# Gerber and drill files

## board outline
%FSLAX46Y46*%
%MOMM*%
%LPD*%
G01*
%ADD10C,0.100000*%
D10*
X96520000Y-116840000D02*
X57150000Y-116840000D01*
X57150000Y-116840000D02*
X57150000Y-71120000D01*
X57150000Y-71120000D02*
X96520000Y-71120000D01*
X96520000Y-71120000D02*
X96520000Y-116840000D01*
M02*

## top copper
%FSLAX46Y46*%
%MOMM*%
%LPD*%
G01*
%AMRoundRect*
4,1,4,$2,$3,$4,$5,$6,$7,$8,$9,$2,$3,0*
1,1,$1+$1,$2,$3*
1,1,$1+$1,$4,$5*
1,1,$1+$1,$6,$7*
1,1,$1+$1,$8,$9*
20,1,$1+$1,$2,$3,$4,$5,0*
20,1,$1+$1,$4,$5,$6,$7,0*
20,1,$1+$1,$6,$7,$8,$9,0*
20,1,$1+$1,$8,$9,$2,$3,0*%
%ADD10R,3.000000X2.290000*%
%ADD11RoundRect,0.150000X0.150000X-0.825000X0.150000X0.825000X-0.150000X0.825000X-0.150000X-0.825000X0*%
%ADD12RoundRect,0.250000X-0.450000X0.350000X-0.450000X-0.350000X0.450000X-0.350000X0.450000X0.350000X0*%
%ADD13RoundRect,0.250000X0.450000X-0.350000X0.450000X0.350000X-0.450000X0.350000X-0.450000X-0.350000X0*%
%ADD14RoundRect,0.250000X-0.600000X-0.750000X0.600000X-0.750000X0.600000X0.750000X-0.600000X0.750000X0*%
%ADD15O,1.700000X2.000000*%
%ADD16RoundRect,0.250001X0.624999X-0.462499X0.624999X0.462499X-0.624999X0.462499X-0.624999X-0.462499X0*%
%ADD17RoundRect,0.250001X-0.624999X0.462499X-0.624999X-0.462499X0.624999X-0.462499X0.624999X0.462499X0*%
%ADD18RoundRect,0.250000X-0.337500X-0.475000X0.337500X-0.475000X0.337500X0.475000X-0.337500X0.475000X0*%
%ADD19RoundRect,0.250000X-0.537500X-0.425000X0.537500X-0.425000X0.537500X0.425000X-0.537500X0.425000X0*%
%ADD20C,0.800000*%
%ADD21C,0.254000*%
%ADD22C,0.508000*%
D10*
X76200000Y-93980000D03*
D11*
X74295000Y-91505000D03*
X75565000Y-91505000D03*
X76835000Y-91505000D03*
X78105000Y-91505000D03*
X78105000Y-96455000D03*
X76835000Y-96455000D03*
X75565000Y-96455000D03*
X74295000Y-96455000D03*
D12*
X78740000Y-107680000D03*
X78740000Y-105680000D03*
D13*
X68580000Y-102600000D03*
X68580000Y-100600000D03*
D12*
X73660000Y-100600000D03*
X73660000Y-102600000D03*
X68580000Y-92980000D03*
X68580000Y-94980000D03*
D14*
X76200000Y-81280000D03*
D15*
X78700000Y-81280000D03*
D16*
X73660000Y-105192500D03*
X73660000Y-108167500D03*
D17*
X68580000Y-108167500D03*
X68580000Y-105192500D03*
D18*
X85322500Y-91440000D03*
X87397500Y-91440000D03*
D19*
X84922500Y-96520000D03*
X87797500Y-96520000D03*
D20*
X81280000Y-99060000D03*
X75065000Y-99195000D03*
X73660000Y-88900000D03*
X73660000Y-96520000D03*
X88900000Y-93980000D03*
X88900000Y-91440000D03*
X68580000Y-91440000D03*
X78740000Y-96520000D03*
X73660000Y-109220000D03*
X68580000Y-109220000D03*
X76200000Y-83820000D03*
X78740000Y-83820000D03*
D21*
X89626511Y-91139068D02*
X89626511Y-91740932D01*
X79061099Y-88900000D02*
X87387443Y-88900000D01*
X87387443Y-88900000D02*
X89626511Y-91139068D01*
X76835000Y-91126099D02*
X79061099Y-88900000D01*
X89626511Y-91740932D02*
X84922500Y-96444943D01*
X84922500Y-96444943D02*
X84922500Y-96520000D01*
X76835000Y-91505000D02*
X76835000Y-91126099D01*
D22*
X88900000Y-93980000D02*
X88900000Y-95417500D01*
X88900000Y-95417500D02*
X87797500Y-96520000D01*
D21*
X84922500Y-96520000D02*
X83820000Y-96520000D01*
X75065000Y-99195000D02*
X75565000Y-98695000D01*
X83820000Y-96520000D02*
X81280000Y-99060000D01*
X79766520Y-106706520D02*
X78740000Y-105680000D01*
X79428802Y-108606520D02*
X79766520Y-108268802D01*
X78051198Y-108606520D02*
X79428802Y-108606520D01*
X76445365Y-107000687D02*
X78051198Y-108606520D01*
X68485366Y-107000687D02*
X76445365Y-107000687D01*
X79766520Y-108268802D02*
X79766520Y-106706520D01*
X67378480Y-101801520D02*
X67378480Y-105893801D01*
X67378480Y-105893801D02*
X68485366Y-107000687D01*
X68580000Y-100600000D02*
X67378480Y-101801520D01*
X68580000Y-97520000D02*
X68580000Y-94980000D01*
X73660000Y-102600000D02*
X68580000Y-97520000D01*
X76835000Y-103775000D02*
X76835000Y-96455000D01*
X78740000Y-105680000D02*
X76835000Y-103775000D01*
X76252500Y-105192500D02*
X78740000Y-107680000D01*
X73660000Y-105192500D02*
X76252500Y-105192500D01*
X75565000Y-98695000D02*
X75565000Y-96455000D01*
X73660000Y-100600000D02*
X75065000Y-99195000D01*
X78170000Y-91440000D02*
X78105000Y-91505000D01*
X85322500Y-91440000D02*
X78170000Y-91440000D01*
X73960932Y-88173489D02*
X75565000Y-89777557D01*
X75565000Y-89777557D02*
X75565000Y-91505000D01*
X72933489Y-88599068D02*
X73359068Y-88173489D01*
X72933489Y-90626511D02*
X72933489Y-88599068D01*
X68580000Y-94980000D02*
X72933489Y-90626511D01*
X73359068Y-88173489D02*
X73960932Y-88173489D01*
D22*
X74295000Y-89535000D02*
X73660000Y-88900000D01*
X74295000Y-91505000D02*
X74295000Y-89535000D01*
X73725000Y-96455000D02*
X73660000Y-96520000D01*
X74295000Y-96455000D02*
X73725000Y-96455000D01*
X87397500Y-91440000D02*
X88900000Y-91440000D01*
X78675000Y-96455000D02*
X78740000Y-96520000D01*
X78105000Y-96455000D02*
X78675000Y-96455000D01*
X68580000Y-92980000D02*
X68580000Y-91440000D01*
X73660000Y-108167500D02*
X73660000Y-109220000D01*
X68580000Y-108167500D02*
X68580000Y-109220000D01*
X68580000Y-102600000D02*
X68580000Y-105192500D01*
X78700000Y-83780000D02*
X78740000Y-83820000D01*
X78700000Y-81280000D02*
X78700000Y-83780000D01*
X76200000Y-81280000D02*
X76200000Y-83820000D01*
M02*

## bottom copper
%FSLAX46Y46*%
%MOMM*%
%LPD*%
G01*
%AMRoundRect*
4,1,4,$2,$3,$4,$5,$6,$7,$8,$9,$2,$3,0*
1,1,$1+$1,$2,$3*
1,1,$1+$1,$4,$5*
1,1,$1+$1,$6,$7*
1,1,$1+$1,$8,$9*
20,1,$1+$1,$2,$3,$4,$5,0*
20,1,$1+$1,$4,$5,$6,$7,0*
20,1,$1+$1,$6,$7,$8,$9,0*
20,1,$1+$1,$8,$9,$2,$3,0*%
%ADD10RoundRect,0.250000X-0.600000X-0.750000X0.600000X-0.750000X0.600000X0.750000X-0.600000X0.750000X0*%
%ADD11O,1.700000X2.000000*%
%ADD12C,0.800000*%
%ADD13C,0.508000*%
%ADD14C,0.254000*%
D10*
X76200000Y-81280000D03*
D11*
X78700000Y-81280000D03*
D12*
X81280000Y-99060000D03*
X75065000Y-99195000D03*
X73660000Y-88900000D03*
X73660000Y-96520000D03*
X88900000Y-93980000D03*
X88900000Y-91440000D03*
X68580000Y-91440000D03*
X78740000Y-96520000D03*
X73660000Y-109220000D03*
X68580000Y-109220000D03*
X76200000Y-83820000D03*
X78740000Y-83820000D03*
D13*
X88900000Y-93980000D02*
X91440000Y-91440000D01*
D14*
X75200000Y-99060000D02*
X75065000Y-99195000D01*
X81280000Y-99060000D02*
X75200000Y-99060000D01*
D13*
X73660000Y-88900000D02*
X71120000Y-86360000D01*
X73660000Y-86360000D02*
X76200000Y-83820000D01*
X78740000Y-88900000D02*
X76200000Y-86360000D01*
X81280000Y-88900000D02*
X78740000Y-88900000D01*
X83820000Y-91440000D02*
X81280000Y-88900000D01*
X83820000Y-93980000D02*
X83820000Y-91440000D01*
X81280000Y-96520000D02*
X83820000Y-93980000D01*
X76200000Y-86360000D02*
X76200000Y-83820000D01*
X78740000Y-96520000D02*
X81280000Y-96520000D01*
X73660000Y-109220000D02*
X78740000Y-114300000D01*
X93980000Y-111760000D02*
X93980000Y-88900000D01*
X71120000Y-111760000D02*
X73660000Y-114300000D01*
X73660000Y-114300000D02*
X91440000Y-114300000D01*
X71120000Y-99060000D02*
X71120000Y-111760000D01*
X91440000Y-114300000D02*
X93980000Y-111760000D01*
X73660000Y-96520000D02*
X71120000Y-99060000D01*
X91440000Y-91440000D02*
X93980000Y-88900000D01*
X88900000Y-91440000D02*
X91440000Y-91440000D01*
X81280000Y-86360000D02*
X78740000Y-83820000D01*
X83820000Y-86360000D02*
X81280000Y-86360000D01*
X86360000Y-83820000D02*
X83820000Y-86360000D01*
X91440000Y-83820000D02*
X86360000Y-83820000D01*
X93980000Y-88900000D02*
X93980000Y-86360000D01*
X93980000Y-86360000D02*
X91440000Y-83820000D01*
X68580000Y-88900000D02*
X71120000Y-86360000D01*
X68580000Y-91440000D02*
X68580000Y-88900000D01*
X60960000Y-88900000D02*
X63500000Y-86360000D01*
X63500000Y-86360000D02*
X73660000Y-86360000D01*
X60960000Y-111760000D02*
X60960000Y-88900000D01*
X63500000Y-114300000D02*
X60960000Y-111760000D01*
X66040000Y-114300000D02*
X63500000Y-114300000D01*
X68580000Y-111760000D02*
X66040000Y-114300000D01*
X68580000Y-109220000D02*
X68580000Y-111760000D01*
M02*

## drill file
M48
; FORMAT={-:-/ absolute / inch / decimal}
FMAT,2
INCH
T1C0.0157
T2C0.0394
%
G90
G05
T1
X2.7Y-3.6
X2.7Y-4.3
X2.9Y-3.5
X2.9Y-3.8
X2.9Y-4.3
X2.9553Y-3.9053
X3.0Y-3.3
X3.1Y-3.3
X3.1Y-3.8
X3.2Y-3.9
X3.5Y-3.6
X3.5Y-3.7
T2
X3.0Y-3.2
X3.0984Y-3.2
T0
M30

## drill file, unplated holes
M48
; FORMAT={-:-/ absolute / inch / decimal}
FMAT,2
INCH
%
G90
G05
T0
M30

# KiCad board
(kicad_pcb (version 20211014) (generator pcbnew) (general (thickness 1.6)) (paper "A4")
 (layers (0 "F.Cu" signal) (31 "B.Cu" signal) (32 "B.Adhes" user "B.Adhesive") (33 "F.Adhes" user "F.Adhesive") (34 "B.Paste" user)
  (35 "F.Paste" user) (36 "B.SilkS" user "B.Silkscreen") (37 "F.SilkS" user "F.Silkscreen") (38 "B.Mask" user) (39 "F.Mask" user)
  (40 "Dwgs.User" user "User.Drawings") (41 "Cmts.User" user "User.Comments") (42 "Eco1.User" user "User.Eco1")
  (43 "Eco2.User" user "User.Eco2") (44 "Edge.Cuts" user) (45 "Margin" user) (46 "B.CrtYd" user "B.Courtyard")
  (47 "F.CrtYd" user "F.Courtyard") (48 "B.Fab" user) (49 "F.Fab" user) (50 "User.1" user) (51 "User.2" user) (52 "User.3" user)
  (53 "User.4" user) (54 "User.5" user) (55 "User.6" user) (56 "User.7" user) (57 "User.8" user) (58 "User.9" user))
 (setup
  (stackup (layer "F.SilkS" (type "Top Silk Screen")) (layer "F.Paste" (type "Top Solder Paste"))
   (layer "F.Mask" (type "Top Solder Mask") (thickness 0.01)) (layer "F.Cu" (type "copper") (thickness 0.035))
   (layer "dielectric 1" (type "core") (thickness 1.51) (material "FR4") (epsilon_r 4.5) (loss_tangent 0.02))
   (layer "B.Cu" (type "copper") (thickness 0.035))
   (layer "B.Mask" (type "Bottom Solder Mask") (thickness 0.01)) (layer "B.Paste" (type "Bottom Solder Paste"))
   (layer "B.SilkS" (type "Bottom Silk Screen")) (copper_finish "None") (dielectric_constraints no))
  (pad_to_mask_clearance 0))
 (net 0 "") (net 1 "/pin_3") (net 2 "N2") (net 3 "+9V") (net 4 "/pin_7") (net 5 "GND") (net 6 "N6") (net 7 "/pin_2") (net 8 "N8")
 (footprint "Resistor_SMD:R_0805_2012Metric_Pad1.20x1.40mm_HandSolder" (layer "F.Cu") (at 78.74 106.68 -90)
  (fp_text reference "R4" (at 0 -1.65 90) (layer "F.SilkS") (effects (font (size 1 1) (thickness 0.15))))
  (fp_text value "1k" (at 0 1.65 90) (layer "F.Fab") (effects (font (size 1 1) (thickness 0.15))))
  (pad "1" smd roundrect (at -1 0 270) (size 1.2 1.4) (layers "F.Cu" "F.Paste" "F.Mask") (roundrect_rratio 0.2083333333) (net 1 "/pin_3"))
  (pad "2" smd roundrect (at 1 0 270) (size 1.2 1.4) (layers "F.Cu" "F.Paste" "F.Mask") (roundrect_rratio 0.2083333333) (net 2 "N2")))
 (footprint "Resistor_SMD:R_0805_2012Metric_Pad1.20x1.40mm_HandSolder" (layer "F.Cu") (at 68.58 93.98 -90)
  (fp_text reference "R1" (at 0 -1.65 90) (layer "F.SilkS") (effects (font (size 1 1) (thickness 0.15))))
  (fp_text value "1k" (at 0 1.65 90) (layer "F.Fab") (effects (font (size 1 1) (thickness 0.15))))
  (pad "1" smd roundrect (at -1 0 270) (size 1.2 1.4) (layers "F.Cu" "F.Paste" "F.Mask") (roundrect_rratio 0.2083333333) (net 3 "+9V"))
  (pad "2" smd roundrect (at 1 0 270) (size 1.2 1.4) (layers "F.Cu" "F.Paste" "F.Mask") (roundrect_rratio 0.2083333333) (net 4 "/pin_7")))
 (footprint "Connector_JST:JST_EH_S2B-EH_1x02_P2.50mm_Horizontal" (layer "F.Cu") (at 76.2 81.28)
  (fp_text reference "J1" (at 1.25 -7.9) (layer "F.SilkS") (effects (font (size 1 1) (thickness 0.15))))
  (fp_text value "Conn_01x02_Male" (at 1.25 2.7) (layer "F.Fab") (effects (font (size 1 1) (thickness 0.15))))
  (pad "1" thru_hole roundrect (at 0 0) (size 1.7 2) (drill 1) (layers *.Cu *.Mask) (roundrect_rratio 0.1470588235) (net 3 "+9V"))
  (pad "2" thru_hole oval (at 2.5 0) (size 1.7 2) (drill 1) (layers *.Cu *.Mask) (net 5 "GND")))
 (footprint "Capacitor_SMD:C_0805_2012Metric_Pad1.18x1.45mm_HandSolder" (layer "F.Cu") (at 86.36 91.44)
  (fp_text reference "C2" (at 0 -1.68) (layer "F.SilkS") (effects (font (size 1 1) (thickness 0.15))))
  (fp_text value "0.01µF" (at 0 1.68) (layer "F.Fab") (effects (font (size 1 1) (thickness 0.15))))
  (pad "1" smd roundrect (at -1.0375 0) (size 1.175 1.45) (layers "F.Cu" "F.Paste" "F.Mask") (roundrect_rratio 0.2127659574) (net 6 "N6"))
  (pad "2" smd roundrect (at 1.0375 0) (size 1.175 1.45) (layers "F.Cu" "F.Paste" "F.Mask") (roundrect_rratio 0.2127659574) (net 5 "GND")))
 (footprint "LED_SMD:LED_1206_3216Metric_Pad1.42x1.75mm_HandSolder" (layer "F.Cu") (at 73.66 106.68 90)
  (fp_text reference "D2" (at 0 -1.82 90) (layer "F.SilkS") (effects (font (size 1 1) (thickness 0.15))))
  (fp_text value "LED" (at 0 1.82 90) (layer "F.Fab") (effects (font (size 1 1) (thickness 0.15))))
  (pad "1" smd roundrect (at -1.4875 0 90) (size 1.425 1.75) (layers "F.Cu" "F.Paste" "F.Mask") (roundrect_rratio 0.1754392982)
   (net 5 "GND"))
  (pad "2" smd roundrect (at 1.4875 0 90) (size 1.425 1.75) (layers "F.Cu" "F.Paste" "F.Mask") (roundrect_rratio 0.1754392982) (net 2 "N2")))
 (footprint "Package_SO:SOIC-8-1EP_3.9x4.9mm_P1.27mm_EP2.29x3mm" (layer "F.Cu") (at 76.2 93.98 90)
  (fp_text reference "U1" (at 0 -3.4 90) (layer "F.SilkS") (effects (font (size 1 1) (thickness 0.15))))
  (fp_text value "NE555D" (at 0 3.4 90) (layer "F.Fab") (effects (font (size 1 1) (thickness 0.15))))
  (pad "" smd roundrect (at 0.57 -0.75 90) (size 0.92 1.21) (layers "F.Paste") (roundrect_rratio 0.25))
  (pad "" smd roundrect (at 0.57 0.75 90) (size 0.92 1.21) (layers "F.Paste") (roundrect_rratio 0.25))
  (pad "" smd roundrect (at -0.57 -0.75 90) (size 0.92 1.21) (layers "F.Paste") (roundrect_rratio 0.25))
  (pad "" smd roundrect (at -0.57 0.75 90) (size 0.92 1.21) (layers "F.Paste") (roundrect_rratio 0.25))
  (pad "1" smd roundrect (at -2.475 -1.905 90) (size 1.95 0.6) (layers "F.Cu" "F.Paste" "F.Mask") (roundrect_rratio 0.25) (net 5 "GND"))
  (pad "2" smd roundrect (at -2.475 -0.635 90) (size 1.95 0.6) (layers "F.Cu" "F.Paste" "F.Mask") (roundrect_rratio 0.25) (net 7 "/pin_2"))
  (pad "3" smd roundrect (at -2.475 0.635 90) (size 1.95 0.6) (layers "F.Cu" "F.Paste" "F.Mask") (roundrect_rratio 0.25) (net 1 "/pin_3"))
  (pad "4" smd roundrect (at -2.475 1.905 90) (size 1.95 0.6) (layers "F.Cu" "F.Paste" "F.Mask") (roundrect_rratio 0.25) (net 3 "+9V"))
  (pad "5" smd roundrect (at 2.475 1.905 90) (size 1.95 0.6) (layers "F.Cu" "F.Paste" "F.Mask") (roundrect_rratio 0.25) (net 6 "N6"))
  (pad "6" smd roundrect (at 2.475 0.635 90) (size 1.95 0.6) (layers "F.Cu" "F.Paste" "F.Mask") (roundrect_rratio 0.25) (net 7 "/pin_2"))
  (pad "7" smd roundrect (at 2.475 -0.635 90) (size 1.95 0.6) (layers "F.Cu" "F.Paste" "F.Mask") (roundrect_rratio 0.25) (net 4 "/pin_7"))
  (pad "8" smd roundrect (at 2.475 -1.905 90) (size 1.95 0.6) (layers "F.Cu" "F.Paste" "F.Mask") (roundrect_rratio 0.25) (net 3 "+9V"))
  (pad "9" smd rect (at 0 0 90) (size 2.29 3) (layers "F.Cu" "F.Mask")))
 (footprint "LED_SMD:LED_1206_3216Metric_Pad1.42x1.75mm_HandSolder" (layer "F.Cu") (at 68.58 106.68 -90)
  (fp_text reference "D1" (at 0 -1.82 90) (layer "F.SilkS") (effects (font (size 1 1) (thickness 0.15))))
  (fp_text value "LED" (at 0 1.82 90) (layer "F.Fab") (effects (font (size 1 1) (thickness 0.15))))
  (pad "1" smd roundrect (at -1.4875 0 270) (size 1.425 1.75) (layers "F.Cu" "F.Paste" "F.Mask") (roundrect_rratio 0.1754392982)
   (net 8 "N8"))
  (pad "2" smd roundrect (at 1.4875 0 270) (size 1.425 1.75) (layers "F.Cu" "F.Paste" "F.Mask") (roundrect_rratio 0.1754392982)
   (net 3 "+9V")))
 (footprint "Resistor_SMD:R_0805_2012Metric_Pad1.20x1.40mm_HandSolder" (layer "F.Cu") (at 68.58 101.6 90)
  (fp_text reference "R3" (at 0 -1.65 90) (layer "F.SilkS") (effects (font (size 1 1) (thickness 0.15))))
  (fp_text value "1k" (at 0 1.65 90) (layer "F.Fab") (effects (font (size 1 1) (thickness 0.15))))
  (pad "1" smd roundrect (at -1 0 90) (size 1.2 1.4) (layers "F.Cu" "F.Paste" "F.Mask") (roundrect_rratio 0.2083333333) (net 8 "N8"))
  (pad "2" smd roundrect (at 1 0 90) (size 1.2 1.4) (layers "F.Cu" "F.Paste" "F.Mask") (roundrect_rratio 0.2083333333) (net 1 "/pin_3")))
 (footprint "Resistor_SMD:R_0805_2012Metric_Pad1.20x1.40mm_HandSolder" (layer "F.Cu") (at 73.66 101.6 -90)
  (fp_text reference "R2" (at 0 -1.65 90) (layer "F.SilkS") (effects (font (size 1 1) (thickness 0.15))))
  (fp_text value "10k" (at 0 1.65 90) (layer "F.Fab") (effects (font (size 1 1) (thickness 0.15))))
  (pad "1" smd roundrect (at -1 0 270) (size 1.2 1.4) (layers "F.Cu" "F.Paste" "F.Mask") (roundrect_rratio 0.2083333333) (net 7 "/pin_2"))
  (pad "2" smd roundrect (at 1 0 270) (size 1.2 1.4) (layers "F.Cu" "F.Paste" "F.Mask") (roundrect_rratio 0.2083333333) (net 4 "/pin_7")))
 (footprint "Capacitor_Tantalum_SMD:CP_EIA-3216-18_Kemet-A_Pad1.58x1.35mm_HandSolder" (layer "F.Cu") (at 86.36 96.52)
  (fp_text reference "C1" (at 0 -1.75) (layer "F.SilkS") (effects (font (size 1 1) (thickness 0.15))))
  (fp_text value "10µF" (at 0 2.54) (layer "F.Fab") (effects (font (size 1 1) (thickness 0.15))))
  (pad "1" smd roundrect (at -1.4375 0) (size 1.575 1.35) (layers "F.Cu" "F.Paste" "F.Mask") (roundrect_rratio 0.1851851852)
   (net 7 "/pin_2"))
  (pad "2" smd roundrect (at 1.4375 0) (size 1.575 1.35) (layers "F.Cu" "F.Paste" "F.Mask") (roundrect_rratio 0.1851851852) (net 5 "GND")))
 (gr_rect (start 96.52 116.84) (end 57.15 71.12) (layer "Edge.Cuts") (width 0.1) (fill none))
 (segment (start 84.9225 96.52) (end 83.82 96.52) (width 0.254) (layer "F.Cu") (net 7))
 (segment (start 89.626511 91.139068) (end 89.626511 91.740932) (width 0.254) (layer "F.Cu") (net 7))
 (segment (start 84.9225 96.444943) (end 84.9225 96.52) (width 0.254) (layer "F.Cu") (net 7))
 (segment (start 73.66 100.6) (end 75.065 99.195) (width 0.254) (layer "F.Cu") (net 7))
 (segment (start 76.835 91.126099) (end 79.061099 88.9) (width 0.254) (layer "F.Cu") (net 7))
 (segment (start 87.387443 88.9) (end 89.626511 91.139068) (width 0.254) (layer "F.Cu") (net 7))
 (segment (start 75.565 98.695) (end 75.565 96.455) (width 0.254) (layer "F.Cu") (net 7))
 (segment (start 89.626511 91.740932) (end 84.9225 96.444943) (width 0.254) (layer "F.Cu") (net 7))
 (segment (start 79.061099 88.9) (end 87.387443 88.9) (width 0.254) (layer "F.Cu") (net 7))
 (segment (start 75.065 99.195) (end 75.565 98.695) (width 0.254) (layer "F.Cu") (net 7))
 (segment (start 83.82 96.52) (end 81.28 99.06) (width 0.254) (layer "F.Cu") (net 7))
 (segment (start 76.835 91.505) (end 76.835 91.126099) (width 0.254) (layer "F.Cu") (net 7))
 (via (at 75.065 99.195) (size 0.8) (drill 0.4) (layers "F.Cu" "B.Cu") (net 7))
 (via (at 81.28 99.06) (size 0.8) (drill 0.4) (layers "F.Cu" "B.Cu") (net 7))
 (segment (start 75.2 99.06) (end 75.065 99.195) (width 0.254) (layer "B.Cu") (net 7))
 (segment (start 81.28 99.06) (end 75.2 99.06) (width 0.254) (layer "B.Cu") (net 7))
 (segment (start 73.725 96.455) (end 73.66 96.52) (width 0.508) (layer "F.Cu") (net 5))
 (segment (start 78.7 83.78) (end 78.74 83.82) (width 0.508) (layer "F.Cu") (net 5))
 (segment (start 87.3975 91.44) (end 88.9 91.44) (width 0.508) (layer "F.Cu") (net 5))
 (segment (start 78.7 81.28) (end 78.7 83.78) (width 0.508) (layer "F.Cu") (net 5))
 (segment (start 88.9 95.4175) (end 87.7975 96.52) (width 0.508) (layer "F.Cu") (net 5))
 (segment (start 73.66 108.1675) (end 73.66 109.22) (width 0.508) (layer "F.Cu") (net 5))
 (segment (start 88.9 93.98) (end 88.9 95.4175) (width 0.508) (layer "F.Cu") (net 5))
 (segment (start 74.295 96.455) (end 73.725 96.455) (width 0.508) (layer "F.Cu") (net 5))
 (via (at 78.74 83.82) (size 0.8) (drill 0.4) (layers "F.Cu" "B.Cu") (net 5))
 (via (at 88.9 91.44) (size 0.8) (drill 0.4) (layers "F.Cu" "B.Cu") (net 5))
 (via (at 73.66 109.22) (size 0.8) (drill 0.4) (layers "F.Cu" "B.Cu") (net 5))
 (via (at 73.66 96.52) (size 0.8) (drill 0.4) (layers "F.Cu" "B.Cu") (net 5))
 (via (at 88.9 93.98) (size 0.8) (drill 0.4) (layers "F.Cu" "B.Cu") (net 5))
 (segment (start 88.9 91.44) (end 91.44 91.44) (width 0.508) (layer "B.Cu") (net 5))
 (segment (start 93.98 111.76) (end 93.98 88.9) (width 0.508) (layer "B.Cu") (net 5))
 (segment (start 73.66 109.22) (end 78.74 114.3) (width 0.508) (layer "B.Cu") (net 5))
 (segment (start 71.12 111.76) (end 73.66 114.3) (width 0.508) (layer "B.Cu") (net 5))
 (segment (start 88.9 93.98) (end 91.44 91.44) (width 0.508) (layer "B.Cu") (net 5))
 (segment (start 73.66 96.52) (end 71.12 99.06) (width 0.508) (layer "B.Cu") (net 5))
 (segment (start 93.98 88.9) (end 93.98 86.36) (width 0.508) (layer "B.Cu") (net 5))
 (segment (start 71.12 99.06) (end 71.12 111.76) (width 0.508) (layer "B.Cu") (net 5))
 (segment (start 86.36 83.82) (end 83.82 86.36) (width 0.508) (layer "B.Cu") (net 5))
 (segment (start 91.44 91.44) (end 93.98 88.9) (width 0.508) (layer "B.Cu") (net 5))
 (segment (start 93.98 86.36) (end 91.44 83.82) (width 0.508) (layer "B.Cu") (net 5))
 (segment (start 81.28 86.36) (end 78.74 83.82) (width 0.508) (layer "B.Cu") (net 5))
 (segment (start 73.66 114.3) (end 91.44 114.3) (width 0.508) (layer "B.Cu") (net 5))
 (segment (start 83.82 86.36) (end 81.28 86.36) (width 0.508) (layer "B.Cu") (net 5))
 (segment (start 91.44 114.3) (end 93.98 111.76) (width 0.508) (layer "B.Cu") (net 5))
 (segment (start 91.44 83.82) (end 86.36 83.82) (width 0.508) (layer "B.Cu") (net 5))
 (segment (start 78.17 91.44) (end 78.105 91.505) (width 0.254) (layer "F.Cu") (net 6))
 (segment (start 85.3225 91.44) (end 78.17 91.44) (width 0.254) (layer "F.Cu") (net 6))
 (segment (start 68.58 102.6) (end 68.58 105.1925) (width 0.508) (layer "F.Cu") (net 8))
 (segment (start 78.105 96.455) (end 78.675 96.455) (width 0.508) (layer "F.Cu") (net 3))
 (segment (start 76.2 81.28) (end 76.2 83.82) (width 0.508) (layer "F.Cu") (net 3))
 (segment (start 78.675 96.455) (end 78.74 96.52) (width 0.508) (layer "F.Cu") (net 3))
 (segment (start 74.295 89.535) (end 73.66 88.9) (width 0.508) (layer "F.Cu") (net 3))
 (segment (start 68.58 92.98) (end 68.58 91.44) (width 0.508) (layer "F.Cu") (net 3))
 (segment (start 68.58 108.1675) (end 68.58 109.22) (width 0.508) (layer "F.Cu") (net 3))
 (segment (start 74.295 91.505) (end 74.295 89.535) (width 0.508) (layer "F.Cu") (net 3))
 (via (at 68.58 91.44) (size 0.8) (drill 0.4) (layers "F.Cu" "B.Cu") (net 3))
 (via (at 73.66 88.9) (size 0.8) (drill 0.4) (layers "F.Cu" "B.Cu") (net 3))
 (via (at 76.2 83.82) (size 0.8) (drill 0.4) (layers "F.Cu" "B.Cu") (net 3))
 (via (at 78.74 96.52) (size 0.8) (drill 0.4) (layers "F.Cu" "B.Cu") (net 3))
 (via (at 68.58 109.22) (size 0.8) (drill 0.4) (layers "F.Cu" "B.Cu") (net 3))
 (segment (start 76.2 86.36) (end 76.2 83.82) (width 0.508) (layer "B.Cu") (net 3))
 (segment (start 81.28 88.9) (end 78.74 88.9) (width 0.508) (layer "B.Cu") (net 3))
 (segment (start 63.5 114.3) (end 60.96 111.76) (width 0.508) (layer "B.Cu") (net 3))
 (segment (start 78.74 96.52) (end 81.28 96.52) (width 0.508) (layer "B.Cu") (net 3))
 (segment (start 83.82 93.98) (end 83.82 91.44) (width 0.508) (layer "B.Cu") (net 3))
 (segment (start 63.5 86.36) (end 73.66 86.36) (width 0.508) (layer "B.Cu") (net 3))
 (segment (start 60.96 88.9) (end 63.5 86.36) (width 0.508) (layer "B.Cu") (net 3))
 (segment (start 68.58 111.76) (end 66.04 114.3) (width 0.508) (layer "B.Cu") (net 3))
 (segment (start 68.58 91.44) (end 68.58 88.9) (width 0.508) (layer "B.Cu") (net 3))
 (segment (start 78.74 88.9) (end 76.2 86.36) (width 0.508) (layer "B.Cu") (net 3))
 (segment (start 68.58 88.9) (end 71.12 86.36) (width 0.508) (layer "B.Cu") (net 3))
 (segment (start 81.28 96.52) (end 83.82 93.98) (width 0.508) (layer "B.Cu") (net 3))
 (segment (start 66.04 114.3) (end 63.5 114.3) (width 0.508) (layer "B.Cu") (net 3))
 (segment (start 68.58 109.22) (end 68.58 111.76) (width 0.508) (layer "B.Cu") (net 3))
 (segment (start 83.82 91.44) (end 81.28 88.9) (width 0.508) (layer "B.Cu") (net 3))
 (segment (start 73.66 88.9) (end 71.12 86.36) (width 0.508) (layer "B.Cu") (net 3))
 (segment (start 73.66 86.36) (end 76.2 83.82) (width 0.508) (layer "B.Cu") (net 3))
 (segment (start 60.96 111.76) (end 60.96 88.9) (width 0.508) (layer "B.Cu") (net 3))
 (segment (start 73.66 105.1925) (end 76.2525 105.1925) (width 0.254) (layer "F.Cu") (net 2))
 (segment (start 76.2525 105.1925) (end 78.74 107.68) (width 0.254) (layer "F.Cu") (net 2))
 (segment (start 72.933489 90.626511) (end 72.933489 88.599068) (width 0.254) (layer "F.Cu") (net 4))
 (segment (start 72.933489 88.599068) (end 73.359068 88.173489) (width 0.254) (layer "F.Cu") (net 4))
 (segment (start 73.66 102.6) (end 68.58 97.52) (width 0.254) (layer "F.Cu") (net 4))
 (segment (start 68.58 94.98) (end 72.933489 90.626511) (width 0.254) (layer "F.Cu") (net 4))
 (segment (start 75.565 89.777557) (end 75.565 91.505) (width 0.254) (layer "F.Cu") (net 4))
 (segment (start 73.359068 88.173489) (end 73.960932 88.173489) (width 0.254) (layer "F.Cu") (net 4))
 (segment (start 68.58 97.52) (end 68.58 94.98) (width 0.254) (layer "F.Cu") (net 4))
 (segment (start 73.960932 88.173489) (end 75.565 89.777557) (width 0.254) (layer "F.Cu") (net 4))
 (segment (start 68.485366 107.000687) (end 76.445365 107.000687) (width 0.254) (layer "F.Cu") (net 1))
 (segment (start 78.74 105.68) (end 76.835 103.775) (width 0.254) (layer "F.Cu") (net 1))
 (segment (start 76.445365 107.000687) (end 78.051198 108.60652) (width 0.254) (layer "F.Cu") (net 1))
 (segment (start 79.76652 106.70652) (end 78.74 105.68) (width 0.254) (layer "F.Cu") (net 1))
 (segment (start 79.428802 108.60652) (end 79.76652 108.268802) (width 0.254) (layer "F.Cu") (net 1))
 (segment (start 78.051198 108.60652) (end 79.428802 108.60652) (width 0.254) (layer "F.Cu") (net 1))
 (segment (start 67.37848 105.893801) (end 68.485366 107.000687) (width 0.254) (layer "F.Cu") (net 1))
 (segment (start 79.76652 108.268802) (end 79.76652 106.70652) (width 0.254) (layer "F.Cu") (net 1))
 (segment (start 67.37848 101.80152) (end 67.37848 105.893801) (width 0.254) (layer "F.Cu") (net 1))
 (segment (start 76.835 103.775) (end 76.835 96.455) (width 0.254) (layer "F.Cu") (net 1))
 (segment (start 68.58 100.6) (end 67.37848 101.80152) (width 0.254) (layer "F.Cu") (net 1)))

